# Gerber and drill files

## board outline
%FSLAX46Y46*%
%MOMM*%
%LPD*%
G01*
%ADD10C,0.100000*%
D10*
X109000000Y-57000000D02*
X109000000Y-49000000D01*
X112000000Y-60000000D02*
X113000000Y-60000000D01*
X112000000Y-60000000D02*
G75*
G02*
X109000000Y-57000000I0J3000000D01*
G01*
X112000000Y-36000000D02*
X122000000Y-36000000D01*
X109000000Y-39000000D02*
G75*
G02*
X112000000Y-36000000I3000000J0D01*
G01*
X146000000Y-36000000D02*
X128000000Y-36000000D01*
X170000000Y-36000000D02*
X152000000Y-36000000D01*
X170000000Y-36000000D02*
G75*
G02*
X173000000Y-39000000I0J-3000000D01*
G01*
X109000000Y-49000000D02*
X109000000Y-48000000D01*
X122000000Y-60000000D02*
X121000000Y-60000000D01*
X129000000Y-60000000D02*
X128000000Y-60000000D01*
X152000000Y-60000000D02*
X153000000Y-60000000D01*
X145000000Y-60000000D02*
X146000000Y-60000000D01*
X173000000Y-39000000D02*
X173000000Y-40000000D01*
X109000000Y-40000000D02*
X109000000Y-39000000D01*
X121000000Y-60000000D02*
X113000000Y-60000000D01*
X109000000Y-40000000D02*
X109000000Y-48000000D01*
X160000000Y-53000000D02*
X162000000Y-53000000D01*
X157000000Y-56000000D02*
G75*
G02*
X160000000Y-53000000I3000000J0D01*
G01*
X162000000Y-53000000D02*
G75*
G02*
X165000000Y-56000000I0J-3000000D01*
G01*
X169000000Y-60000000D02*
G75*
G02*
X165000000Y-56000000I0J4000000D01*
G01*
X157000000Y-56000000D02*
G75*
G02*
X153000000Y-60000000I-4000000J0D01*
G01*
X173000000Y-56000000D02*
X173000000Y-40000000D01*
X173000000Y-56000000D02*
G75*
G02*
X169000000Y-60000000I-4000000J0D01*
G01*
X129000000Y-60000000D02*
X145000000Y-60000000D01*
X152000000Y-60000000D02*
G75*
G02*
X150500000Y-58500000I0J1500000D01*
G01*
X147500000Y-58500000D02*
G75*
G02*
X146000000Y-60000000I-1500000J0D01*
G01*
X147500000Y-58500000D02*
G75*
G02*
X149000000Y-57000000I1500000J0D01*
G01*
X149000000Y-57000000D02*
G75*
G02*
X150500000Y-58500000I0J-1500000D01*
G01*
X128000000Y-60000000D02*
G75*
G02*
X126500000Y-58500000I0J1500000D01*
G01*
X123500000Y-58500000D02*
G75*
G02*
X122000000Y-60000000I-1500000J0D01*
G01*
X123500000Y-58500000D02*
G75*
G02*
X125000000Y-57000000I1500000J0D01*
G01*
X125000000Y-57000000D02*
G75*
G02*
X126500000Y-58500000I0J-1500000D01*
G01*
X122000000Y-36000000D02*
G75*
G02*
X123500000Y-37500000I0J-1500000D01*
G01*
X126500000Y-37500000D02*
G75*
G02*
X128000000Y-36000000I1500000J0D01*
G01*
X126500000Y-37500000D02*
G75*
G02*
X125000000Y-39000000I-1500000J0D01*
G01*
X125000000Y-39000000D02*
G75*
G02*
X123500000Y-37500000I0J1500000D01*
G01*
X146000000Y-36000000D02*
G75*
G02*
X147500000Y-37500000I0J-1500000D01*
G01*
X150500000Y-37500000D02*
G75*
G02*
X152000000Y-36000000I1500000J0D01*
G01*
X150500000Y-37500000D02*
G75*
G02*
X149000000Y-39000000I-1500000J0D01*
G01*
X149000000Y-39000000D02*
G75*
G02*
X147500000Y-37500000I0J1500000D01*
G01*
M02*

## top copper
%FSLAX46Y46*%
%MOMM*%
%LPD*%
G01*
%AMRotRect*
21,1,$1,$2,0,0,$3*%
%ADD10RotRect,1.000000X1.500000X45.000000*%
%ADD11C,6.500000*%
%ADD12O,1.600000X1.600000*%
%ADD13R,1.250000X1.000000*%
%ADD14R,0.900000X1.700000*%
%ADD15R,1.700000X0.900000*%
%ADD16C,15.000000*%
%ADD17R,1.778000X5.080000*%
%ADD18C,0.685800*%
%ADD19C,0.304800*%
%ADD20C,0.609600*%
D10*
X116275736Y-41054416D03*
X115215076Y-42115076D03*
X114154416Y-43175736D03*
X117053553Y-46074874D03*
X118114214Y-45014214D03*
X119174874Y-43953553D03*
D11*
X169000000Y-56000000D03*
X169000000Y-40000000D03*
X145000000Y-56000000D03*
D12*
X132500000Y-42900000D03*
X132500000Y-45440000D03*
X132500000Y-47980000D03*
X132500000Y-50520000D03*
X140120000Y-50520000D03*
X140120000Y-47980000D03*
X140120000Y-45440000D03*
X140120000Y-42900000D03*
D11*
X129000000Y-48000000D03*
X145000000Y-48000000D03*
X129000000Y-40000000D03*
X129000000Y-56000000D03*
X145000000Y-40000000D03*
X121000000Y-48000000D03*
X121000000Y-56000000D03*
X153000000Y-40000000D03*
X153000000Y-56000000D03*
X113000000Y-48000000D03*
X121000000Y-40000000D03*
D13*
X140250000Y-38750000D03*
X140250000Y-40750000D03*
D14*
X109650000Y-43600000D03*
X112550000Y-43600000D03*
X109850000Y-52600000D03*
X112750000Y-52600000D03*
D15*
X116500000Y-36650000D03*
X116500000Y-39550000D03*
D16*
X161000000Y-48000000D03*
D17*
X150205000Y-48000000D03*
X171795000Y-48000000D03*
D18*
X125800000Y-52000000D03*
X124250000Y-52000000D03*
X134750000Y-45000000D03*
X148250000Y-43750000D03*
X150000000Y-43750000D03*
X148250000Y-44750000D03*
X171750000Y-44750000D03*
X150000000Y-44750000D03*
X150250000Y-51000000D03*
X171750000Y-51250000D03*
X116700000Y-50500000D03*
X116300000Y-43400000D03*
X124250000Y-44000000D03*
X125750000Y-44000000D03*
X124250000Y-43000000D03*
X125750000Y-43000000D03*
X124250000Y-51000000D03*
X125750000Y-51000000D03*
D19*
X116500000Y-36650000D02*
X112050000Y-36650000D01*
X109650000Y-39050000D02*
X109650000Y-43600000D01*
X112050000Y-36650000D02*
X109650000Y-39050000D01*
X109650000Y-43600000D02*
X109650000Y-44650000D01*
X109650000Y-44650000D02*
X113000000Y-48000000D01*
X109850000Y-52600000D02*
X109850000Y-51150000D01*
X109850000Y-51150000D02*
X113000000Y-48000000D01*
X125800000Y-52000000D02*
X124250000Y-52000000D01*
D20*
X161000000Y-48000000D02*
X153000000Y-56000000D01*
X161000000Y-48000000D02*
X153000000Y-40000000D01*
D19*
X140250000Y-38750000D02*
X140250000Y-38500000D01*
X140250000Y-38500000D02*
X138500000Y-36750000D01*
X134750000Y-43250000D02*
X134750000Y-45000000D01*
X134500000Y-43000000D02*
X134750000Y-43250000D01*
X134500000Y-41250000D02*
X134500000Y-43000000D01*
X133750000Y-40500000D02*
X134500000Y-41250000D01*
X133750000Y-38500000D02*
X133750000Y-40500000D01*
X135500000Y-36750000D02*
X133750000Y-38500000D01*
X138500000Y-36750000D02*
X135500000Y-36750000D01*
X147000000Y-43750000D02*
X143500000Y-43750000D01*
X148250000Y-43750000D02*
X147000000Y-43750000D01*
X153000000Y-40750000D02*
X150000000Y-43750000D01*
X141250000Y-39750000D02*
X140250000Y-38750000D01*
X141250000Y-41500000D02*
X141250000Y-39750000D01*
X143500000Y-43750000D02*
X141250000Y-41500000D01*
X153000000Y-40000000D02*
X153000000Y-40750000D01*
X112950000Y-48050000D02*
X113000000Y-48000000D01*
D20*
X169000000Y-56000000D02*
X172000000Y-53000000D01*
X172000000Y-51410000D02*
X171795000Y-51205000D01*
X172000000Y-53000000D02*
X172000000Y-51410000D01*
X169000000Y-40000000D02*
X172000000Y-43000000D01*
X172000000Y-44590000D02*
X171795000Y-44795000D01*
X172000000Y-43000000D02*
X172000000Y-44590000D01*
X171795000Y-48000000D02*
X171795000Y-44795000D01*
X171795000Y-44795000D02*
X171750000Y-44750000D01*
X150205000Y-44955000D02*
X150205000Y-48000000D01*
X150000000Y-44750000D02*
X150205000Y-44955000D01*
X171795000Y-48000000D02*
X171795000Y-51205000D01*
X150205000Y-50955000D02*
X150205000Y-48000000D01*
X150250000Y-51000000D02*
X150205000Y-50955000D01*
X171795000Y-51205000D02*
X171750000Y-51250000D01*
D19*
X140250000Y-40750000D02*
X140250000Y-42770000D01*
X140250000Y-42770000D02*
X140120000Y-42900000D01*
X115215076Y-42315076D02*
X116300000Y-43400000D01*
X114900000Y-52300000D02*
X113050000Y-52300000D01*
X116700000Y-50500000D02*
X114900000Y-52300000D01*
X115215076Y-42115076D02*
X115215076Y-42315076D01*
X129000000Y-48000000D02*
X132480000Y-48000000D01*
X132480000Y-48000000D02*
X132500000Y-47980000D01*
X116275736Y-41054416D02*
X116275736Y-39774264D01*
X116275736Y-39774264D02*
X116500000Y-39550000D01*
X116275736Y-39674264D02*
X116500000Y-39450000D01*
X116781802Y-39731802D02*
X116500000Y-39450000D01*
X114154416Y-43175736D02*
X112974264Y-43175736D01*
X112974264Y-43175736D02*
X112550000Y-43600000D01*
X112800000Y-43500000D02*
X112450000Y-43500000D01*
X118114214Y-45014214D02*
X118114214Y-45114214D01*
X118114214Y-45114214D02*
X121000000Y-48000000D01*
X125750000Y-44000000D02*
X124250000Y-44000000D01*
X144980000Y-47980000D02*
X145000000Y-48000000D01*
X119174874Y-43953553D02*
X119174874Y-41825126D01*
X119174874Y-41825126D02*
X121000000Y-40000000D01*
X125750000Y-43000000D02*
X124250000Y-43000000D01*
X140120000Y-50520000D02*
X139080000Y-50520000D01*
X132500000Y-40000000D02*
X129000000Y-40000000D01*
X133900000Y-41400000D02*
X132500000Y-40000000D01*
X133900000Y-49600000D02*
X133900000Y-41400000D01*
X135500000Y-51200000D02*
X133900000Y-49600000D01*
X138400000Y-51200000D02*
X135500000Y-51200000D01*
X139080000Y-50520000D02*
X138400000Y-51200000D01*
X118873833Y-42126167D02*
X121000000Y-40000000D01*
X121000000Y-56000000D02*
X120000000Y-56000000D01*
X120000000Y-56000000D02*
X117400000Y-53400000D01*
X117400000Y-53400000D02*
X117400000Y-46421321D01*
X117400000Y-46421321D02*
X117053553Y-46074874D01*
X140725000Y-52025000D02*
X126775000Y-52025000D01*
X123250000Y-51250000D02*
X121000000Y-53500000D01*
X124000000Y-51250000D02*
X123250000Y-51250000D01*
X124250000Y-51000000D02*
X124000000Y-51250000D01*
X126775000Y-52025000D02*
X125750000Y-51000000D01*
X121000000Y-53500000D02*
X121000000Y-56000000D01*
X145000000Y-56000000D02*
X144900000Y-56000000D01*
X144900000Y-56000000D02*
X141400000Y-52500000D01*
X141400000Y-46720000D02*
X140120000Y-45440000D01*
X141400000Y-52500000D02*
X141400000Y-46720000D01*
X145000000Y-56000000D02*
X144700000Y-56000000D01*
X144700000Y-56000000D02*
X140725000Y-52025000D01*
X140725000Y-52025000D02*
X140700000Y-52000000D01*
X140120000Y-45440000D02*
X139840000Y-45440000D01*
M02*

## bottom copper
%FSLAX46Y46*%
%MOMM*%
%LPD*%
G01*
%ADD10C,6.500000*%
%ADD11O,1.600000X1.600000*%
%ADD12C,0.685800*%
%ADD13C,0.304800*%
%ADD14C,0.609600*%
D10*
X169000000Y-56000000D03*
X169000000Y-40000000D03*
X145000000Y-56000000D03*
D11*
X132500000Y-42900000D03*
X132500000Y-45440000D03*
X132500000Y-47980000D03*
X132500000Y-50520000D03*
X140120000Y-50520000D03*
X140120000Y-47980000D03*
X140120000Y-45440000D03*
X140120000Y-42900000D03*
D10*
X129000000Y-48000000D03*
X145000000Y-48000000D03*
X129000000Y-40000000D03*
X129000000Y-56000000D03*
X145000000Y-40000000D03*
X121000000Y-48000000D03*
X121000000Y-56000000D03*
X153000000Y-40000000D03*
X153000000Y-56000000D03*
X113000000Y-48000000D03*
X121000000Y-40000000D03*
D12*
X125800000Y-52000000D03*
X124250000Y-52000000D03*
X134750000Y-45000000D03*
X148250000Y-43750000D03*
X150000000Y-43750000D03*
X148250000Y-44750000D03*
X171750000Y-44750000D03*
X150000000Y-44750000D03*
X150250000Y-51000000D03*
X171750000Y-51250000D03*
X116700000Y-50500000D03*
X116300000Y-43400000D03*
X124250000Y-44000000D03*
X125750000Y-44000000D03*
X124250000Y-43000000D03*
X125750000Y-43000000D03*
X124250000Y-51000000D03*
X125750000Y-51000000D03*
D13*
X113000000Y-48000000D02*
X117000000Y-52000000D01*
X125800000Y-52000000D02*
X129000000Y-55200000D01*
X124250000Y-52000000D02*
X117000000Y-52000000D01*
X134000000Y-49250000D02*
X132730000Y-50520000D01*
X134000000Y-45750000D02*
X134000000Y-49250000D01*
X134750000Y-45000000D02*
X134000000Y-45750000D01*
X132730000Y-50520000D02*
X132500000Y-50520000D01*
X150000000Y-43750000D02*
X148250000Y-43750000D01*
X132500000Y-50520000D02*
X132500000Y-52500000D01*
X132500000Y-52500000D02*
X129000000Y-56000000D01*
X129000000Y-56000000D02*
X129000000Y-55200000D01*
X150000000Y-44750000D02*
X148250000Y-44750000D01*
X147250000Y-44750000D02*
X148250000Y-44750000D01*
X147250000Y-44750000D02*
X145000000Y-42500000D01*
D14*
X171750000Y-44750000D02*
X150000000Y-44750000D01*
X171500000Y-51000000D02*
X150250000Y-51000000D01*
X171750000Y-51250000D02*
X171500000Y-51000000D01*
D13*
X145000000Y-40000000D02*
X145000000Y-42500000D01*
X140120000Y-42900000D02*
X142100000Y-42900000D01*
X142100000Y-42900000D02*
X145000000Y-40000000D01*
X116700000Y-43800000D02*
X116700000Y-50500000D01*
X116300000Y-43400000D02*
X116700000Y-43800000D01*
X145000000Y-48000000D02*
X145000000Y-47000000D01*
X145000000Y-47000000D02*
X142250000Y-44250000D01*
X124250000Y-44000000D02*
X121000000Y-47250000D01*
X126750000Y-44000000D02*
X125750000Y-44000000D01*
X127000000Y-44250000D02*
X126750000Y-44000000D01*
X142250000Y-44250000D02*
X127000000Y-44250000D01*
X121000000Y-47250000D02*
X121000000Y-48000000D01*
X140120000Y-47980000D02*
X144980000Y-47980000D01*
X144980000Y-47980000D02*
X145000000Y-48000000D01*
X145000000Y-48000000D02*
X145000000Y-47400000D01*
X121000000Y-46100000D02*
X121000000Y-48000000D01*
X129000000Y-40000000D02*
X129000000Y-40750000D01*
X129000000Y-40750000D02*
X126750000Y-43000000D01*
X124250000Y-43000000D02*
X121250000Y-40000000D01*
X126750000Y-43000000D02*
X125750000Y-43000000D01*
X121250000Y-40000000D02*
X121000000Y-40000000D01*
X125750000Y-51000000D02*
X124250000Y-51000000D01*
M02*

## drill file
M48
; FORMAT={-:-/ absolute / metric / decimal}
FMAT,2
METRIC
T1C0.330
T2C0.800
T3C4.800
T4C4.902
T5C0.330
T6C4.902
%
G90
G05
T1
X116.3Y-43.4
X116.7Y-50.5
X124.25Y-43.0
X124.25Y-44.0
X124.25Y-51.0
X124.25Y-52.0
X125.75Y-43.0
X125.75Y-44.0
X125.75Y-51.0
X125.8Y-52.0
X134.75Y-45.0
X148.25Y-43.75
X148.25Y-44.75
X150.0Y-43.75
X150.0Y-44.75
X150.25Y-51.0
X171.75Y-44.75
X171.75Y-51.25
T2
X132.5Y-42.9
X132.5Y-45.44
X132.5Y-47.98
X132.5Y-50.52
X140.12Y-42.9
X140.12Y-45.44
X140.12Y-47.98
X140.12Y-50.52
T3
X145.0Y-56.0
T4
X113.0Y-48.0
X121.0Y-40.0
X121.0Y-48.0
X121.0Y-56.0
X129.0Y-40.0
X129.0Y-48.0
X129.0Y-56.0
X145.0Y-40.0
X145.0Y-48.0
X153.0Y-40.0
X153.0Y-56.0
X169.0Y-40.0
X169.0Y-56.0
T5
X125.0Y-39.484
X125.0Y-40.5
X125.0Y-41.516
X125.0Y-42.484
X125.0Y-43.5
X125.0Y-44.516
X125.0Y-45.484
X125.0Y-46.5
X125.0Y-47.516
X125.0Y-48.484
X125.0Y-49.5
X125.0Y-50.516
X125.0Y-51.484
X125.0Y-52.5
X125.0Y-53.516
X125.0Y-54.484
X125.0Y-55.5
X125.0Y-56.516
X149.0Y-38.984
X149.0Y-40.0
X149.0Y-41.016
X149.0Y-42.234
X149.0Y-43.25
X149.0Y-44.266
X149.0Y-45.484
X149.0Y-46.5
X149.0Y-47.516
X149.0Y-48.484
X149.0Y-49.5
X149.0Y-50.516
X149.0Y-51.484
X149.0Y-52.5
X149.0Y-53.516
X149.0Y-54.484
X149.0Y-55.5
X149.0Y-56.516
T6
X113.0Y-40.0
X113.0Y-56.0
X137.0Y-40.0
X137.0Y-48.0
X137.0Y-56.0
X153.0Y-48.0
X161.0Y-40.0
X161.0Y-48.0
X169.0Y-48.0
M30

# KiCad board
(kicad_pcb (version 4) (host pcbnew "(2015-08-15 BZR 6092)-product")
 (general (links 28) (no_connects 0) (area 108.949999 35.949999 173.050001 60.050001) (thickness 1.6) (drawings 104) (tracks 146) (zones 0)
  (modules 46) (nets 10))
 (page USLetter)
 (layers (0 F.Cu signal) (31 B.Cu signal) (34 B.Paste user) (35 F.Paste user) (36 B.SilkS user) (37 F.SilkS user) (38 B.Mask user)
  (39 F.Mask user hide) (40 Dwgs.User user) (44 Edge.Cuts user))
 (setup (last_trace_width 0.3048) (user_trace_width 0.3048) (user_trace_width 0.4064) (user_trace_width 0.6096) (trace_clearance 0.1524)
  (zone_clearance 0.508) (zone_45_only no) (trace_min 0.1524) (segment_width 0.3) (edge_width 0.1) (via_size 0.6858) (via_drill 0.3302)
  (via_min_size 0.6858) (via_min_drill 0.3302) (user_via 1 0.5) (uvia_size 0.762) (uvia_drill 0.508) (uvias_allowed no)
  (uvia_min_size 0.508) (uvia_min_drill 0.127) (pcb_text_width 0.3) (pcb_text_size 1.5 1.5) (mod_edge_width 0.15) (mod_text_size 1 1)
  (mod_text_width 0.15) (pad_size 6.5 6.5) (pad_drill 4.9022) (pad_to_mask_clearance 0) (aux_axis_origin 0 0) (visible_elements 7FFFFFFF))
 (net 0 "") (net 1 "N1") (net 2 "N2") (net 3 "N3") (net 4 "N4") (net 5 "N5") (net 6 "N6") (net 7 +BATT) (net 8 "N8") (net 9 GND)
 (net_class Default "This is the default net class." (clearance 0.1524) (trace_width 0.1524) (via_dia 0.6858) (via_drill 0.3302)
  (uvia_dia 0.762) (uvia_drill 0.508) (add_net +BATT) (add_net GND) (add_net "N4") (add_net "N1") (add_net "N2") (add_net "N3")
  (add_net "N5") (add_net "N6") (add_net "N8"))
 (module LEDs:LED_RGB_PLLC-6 (layer F.Cu) (at 116.7 43.6 315)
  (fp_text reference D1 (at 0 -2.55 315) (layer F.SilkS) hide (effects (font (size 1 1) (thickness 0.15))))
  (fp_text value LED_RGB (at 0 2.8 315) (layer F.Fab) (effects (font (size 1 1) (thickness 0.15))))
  (pad 1 smd rect (at -2.1 -1.5 45) (size 1 1.5) (layers F.Cu F.Paste F.Mask) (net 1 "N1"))
  (pad 2 smd rect (at -2.1 0 45) (size 1 1.5) (layers F.Cu F.Paste F.Mask) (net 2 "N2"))
  (pad 3 smd rect (at -2.1 1.5 45) (size 1 1.5) (layers F.Cu F.Paste F.Mask) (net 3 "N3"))
  (pad 4 smd rect (at 2 1.5 45) (size 1 1.5) (layers F.Cu F.Paste F.Mask) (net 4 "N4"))
  (pad 5 smd rect (at 2 0 45) (size 1 1.5) (layers F.Cu F.Paste F.Mask) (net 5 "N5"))
  (pad 6 smd rect (at 2 -1.5 45) (size 1 1.5) (layers F.Cu F.Paste F.Mask) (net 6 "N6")))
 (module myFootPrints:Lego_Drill (layer F.Cu) (at 113 40)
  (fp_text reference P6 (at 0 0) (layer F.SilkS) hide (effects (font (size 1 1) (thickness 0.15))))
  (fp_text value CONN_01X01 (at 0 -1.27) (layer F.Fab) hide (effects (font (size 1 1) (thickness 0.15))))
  (pad "" np_thru_hole circle (at 0 0) (size 4.9022 4.9022) (drill 4.9022) (layers *.Cu *.Mask F.SilkS)))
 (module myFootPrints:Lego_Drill (layer F.Cu) (at 113 56)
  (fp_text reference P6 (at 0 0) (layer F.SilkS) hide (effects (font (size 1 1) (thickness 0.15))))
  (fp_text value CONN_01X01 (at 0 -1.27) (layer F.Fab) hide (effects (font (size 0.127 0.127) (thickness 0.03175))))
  (pad "" np_thru_hole circle (at 0 0) (size 4.9022 4.9022) (drill 4.9022) (layers *.Cu *.Mask F.SilkS)))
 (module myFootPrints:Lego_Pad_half (layer F.Cu) (at 169 56 180)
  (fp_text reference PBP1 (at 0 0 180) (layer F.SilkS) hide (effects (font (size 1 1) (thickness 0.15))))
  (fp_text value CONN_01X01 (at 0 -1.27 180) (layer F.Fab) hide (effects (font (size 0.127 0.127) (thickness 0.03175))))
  (pad 1 thru_hole circle (at 0 0 180) (size 6.5 6.5) (drill 4.9022) (layers *.Cu B.Mask) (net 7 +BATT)))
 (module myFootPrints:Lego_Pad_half (layer F.Cu) (at 169 40 270)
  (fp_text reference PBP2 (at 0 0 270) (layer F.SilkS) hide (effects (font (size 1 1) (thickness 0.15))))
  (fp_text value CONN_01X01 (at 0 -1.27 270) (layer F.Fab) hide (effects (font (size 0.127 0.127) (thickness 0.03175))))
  (pad 1 thru_hole circle (at 0 0 270) (size 6.5 6.5) (drill 4.9022) (layers *.Cu B.Mask) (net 7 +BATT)))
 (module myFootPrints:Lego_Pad (layer F.Cu) (at 145 56)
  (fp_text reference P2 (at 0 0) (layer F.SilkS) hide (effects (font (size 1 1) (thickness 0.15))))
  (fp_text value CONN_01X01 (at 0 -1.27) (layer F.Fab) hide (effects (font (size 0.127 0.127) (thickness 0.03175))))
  (pad 1 thru_hole circle (at 0 0) (size 6.5 6.5) (drill 4.8) (layers *.Cu *.Mask F.SilkS) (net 4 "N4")))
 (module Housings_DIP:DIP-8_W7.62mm (layer F.Cu) (at 132.5 42.9)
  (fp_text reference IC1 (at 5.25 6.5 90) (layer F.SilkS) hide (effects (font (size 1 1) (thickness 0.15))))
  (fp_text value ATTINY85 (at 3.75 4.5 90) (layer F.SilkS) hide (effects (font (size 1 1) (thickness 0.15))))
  (pad 1 thru_hole oval (at 0 0) (size 1.6 1.6) (drill 0.8) (layers *.Cu *.Mask F.SilkS))
  (pad 2 thru_hole oval (at 0 2.54) (size 1.6 1.6) (drill 0.8) (layers *.Cu *.Mask F.SilkS))
  (pad 3 thru_hole oval (at 0 5.08) (size 1.6 1.6) (drill 0.8) (layers *.Cu *.Mask F.SilkS) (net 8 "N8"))
  (pad 4 thru_hole oval (at 0 7.62) (size 1.6 1.6) (drill 0.8) (layers *.Cu *.Mask F.SilkS) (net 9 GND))
  (pad 5 thru_hole oval (at 7.62 7.62) (size 1.6 1.6) (drill 0.8) (layers *.Cu *.Mask F.SilkS) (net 6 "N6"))
  (pad 6 thru_hole oval (at 7.62 5.08) (size 1.6 1.6) (drill 0.8) (layers *.Cu *.Mask F.SilkS) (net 5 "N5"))
  (pad 7 thru_hole oval (at 7.62 2.54) (size 1.6 1.6) (drill 0.8) (layers *.Cu *.Mask F.SilkS) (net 4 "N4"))
  (pad 8 thru_hole oval (at 7.62 0) (size 1.6 1.6) (drill 0.8) (layers *.Cu *.Mask F.SilkS) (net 7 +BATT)))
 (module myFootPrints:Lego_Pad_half (layer F.Cu) (at 129 48 45)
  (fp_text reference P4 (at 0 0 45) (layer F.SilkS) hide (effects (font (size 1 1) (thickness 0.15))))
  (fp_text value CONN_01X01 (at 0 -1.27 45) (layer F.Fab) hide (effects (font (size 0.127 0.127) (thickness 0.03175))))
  (pad 1 thru_hole circle (at 0 0 45) (size 6.5 6.5) (drill 4.9022) (layers *.Cu *.Mask F.SilkS) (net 8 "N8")))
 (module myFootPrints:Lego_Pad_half (layer F.Cu) (at 145 48 225)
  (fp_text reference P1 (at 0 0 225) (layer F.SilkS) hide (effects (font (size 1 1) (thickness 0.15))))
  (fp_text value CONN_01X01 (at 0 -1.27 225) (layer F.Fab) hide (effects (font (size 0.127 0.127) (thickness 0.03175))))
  (pad 1 thru_hole circle (at 0 0 225) (size 6.5 6.5) (drill 4.9022) (layers *.Cu *.Mask F.SilkS) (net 5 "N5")))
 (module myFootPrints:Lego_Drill (layer F.Cu) (at 137 40)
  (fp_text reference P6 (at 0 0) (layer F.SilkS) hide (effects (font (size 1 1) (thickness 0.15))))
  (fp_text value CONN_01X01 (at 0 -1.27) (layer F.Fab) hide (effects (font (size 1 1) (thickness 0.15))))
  (pad "" np_thru_hole circle (at 0 0) (size 4.9022 4.9022) (drill 4.9022) (layers *.Cu *.Mask F.SilkS)))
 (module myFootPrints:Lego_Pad (layer F.Cu) (at 129 40)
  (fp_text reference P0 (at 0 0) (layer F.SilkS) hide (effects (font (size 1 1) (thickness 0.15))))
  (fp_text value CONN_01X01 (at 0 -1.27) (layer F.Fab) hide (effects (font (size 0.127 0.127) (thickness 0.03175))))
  (pad 1 thru_hole circle (at 0 0) (size 6.5 6.5) (drill 4.9022) (layers *.Cu *.Mask F.SilkS) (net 6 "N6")))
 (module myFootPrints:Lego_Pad (layer F.Cu) (at 129 56)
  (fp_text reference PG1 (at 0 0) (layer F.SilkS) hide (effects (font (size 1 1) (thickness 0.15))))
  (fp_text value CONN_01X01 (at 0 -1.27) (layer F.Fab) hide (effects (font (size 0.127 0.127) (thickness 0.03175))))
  (pad 1 thru_hole circle (at 0 0) (size 6.5 6.5) (drill 4.9022) (layers *.Cu *.Mask F.SilkS) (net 9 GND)))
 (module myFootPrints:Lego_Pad (layer F.Cu) (at 145 40)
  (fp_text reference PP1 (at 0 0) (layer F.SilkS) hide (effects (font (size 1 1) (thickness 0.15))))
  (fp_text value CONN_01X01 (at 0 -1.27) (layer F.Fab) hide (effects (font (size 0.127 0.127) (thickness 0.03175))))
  (pad 1 thru_hole circle (at 0 0) (size 6.5 6.5) (drill 4.9022) (layers *.Cu *.Mask F.SilkS) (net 7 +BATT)))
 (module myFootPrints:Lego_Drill (layer F.Cu) (at 137 48)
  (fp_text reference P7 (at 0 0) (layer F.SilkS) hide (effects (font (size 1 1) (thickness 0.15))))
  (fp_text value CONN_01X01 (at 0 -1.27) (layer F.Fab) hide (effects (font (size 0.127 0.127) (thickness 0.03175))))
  (pad "" np_thru_hole circle (at 0 0) (size 4.9022 4.9022) (drill 4.9022) (layers *.Cu *.Mask F.SilkS)))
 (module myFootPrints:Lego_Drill (layer F.Cu) (at 137 56)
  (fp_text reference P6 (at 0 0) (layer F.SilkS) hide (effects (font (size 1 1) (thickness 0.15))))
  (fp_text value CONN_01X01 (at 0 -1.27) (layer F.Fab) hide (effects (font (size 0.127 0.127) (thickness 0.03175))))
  (pad "" np_thru_hole circle (at 0 0) (size 4.9022 4.9022) (drill 4.9022) (layers *.Cu *.Mask F.SilkS)))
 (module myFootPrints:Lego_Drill (layer F.Cu) (at 161 48)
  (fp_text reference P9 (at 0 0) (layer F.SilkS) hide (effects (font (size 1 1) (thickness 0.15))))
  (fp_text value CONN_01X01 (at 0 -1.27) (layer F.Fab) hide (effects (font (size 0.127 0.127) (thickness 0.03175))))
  (pad "" np_thru_hole circle (at 0 0) (size 4.9022 4.9022) (drill 4.9022) (layers *.Cu *.Mask F.SilkS)))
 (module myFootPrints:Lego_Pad (layer F.Cu) (at 121 48)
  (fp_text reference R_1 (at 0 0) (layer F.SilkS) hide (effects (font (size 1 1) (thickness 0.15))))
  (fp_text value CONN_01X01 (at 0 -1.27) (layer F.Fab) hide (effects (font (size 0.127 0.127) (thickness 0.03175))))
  (pad 1 thru_hole circle (at 0 0) (size 6.5 6.5) (drill 4.9022) (layers *.Cu *.Mask F.SilkS) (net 5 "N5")))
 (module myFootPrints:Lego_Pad (layer F.Cu) (at 121 56)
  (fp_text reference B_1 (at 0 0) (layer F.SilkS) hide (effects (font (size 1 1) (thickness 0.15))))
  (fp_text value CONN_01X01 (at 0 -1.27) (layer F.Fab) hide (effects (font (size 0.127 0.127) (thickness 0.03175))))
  (pad 1 thru_hole circle (at 0 0) (size 6.5 6.5) (drill 4.9022) (layers *.Cu *.Mask F.SilkS) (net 4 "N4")))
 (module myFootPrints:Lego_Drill (layer F.Cu) (at 169 48)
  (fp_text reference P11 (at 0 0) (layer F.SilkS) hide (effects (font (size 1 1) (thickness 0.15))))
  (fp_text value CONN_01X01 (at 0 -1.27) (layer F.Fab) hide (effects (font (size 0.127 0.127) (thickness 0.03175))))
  (pad "" np_thru_hole circle (at 0 0) (size 4.9022 4.9022) (drill 4.9022) (layers *.Cu *.Mask F.SilkS)))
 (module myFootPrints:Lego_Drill (layer F.Cu) (at 153 48)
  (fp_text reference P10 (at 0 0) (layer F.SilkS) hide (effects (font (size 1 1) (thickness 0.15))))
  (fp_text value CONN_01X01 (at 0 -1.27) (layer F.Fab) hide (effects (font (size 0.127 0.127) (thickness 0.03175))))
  (pad "" np_thru_hole circle (at 0 0) (size 4.9022 4.9022) (drill 4.9022) (layers *.Cu *.Mask F.SilkS)))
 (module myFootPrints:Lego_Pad (layer F.Cu) (at 153 40)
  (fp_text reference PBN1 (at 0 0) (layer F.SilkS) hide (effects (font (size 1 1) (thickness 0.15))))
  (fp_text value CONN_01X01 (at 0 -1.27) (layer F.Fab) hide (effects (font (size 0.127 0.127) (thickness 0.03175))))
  (pad 1 thru_hole circle (at 0 0) (size 6.5 6.5) (drill 4.9022) (layers *.Cu *.Mask F.SilkS) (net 9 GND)))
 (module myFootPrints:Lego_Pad (layer F.Cu) (at 153 56)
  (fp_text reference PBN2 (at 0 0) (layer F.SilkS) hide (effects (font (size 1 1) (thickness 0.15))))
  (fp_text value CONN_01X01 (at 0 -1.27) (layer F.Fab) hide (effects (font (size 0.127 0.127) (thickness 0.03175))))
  (pad 1 thru_hole circle (at 0 0) (size 6.5 6.5) (drill 4.9022) (layers *.Cu *.Mask F.SilkS) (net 9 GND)))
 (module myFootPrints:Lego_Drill (layer F.Cu) (at 161 40)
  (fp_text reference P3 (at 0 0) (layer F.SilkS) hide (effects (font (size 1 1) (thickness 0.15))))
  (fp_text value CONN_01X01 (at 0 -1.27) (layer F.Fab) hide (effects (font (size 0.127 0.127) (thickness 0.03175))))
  (pad "" np_thru_hole circle (at 0 0) (size 4.9022 4.9022) (drill 4.9022) (layers *.Cu *.Mask F.SilkS)))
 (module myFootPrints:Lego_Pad (layer F.Cu) (at 113 48)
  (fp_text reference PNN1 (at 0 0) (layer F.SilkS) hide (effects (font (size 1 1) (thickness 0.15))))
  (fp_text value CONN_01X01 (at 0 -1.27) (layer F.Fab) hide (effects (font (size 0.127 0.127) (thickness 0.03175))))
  (pad 1 thru_hole circle (at 0 0) (size 6.5 6.5) (drill 4.9022) (layers *.Cu *.Mask F.SilkS) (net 9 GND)))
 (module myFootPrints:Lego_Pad (layer F.Cu) (at 121 40)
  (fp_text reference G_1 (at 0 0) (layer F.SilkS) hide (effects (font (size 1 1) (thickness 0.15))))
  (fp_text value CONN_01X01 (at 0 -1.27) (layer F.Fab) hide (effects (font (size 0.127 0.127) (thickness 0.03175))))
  (pad 1 thru_hole circle (at 0 0) (size 6.5 6.5) (drill 4.9022) (layers *.Cu *.Mask F.SilkS) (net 6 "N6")))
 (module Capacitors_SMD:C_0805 (layer F.Cu) (at 140.25 39.75 270)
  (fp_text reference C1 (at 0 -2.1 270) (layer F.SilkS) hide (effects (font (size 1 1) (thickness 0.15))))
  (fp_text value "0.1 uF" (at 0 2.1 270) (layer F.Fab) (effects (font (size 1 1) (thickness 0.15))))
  (pad 1 smd rect (at -1 0 270) (size 1 1.25) (layers F.Cu F.Paste F.Mask) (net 9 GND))
  (pad 2 smd rect (at 1 0 270) (size 1 1.25) (layers F.Cu F.Paste F.Mask) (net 7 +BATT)))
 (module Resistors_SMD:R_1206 (layer F.Cu) (at 111.1 43.6)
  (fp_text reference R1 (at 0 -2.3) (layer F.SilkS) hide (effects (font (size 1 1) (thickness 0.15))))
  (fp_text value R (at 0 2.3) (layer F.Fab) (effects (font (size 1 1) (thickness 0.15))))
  (pad 1 smd rect (at -1.45 0) (size 0.9 1.7) (layers F.Cu F.Paste F.Mask) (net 9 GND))
  (pad 2 smd rect (at 1.45 0) (size 0.9 1.7) (layers F.Cu F.Paste F.Mask) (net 3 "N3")))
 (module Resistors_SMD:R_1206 (layer F.Cu) (at 111.3 52.6)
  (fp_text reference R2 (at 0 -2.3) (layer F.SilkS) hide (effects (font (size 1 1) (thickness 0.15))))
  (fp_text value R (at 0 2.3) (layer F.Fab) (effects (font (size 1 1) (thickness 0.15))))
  (pad 1 smd rect (at -1.45 0) (size 0.9 1.7) (layers F.Cu F.Paste F.Mask) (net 9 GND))
  (pad 2 smd rect (at 1.45 0) (size 0.9 1.7) (layers F.Cu F.Paste F.Mask) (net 2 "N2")))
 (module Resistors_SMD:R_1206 (layer F.Cu) (at 116.5 38.1 270)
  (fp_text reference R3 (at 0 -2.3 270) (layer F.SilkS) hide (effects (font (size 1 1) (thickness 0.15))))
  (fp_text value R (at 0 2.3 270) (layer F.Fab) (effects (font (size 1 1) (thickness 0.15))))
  (pad 1 smd rect (at -1.45 0 270) (size 0.9 1.7) (layers F.Cu F.Paste F.Mask) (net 9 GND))
  (pad 2 smd rect (at 1.45 0 270) (size 0.9 1.7) (layers F.Cu F.Paste F.Mask) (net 1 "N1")))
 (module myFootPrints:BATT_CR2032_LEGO (layer F.Cu) (at 161 48)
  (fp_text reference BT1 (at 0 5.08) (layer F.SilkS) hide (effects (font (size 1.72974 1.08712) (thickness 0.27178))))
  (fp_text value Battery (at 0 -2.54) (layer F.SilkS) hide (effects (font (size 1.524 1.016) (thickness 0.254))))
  (pad 2 smd circle (at 0 0) (size 15 15) (layers F.Cu F.Paste F.Mask) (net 9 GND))
  (pad 1 smd rect (at -10.795 0) (size 1.778 5.08) (layers F.Cu F.Paste F.Mask) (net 7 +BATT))
  (pad 1 smd rect (at 10.795 0) (size 1.778 5.08) (layers F.Cu F.Paste F.Mask) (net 7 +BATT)))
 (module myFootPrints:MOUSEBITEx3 (layer F.Cu) (at 149 40 90)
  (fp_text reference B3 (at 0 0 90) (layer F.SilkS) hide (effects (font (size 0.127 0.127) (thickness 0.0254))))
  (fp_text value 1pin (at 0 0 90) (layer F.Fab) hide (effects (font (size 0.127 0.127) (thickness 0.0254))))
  (pad "" np_thru_hole circle (at -1.016 0 90) (size 0.3302 0.3302) (drill 0.3302) (layers *.Cu *.Mask F.SilkS))
  (pad "" np_thru_hole circle (at 1.016 0 90) (size 0.3302 0.3302) (drill 0.3302) (layers *.Cu *.Mask F.SilkS))
  (pad "" np_thru_hole circle (at 0 0 90) (size 0.3302 0.3302) (drill 0.3302) (layers *.Cu *.Mask F.SilkS)))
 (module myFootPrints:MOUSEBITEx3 (layer F.Cu) (at 149 49.5 90)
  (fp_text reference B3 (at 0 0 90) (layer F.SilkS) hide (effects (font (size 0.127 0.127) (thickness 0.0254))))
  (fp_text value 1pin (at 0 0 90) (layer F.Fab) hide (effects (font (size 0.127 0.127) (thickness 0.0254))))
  (pad "" np_thru_hole circle (at -1.016 0 90) (size 0.3302 0.3302) (drill 0.3302) (layers *.Cu *.Mask F.SilkS))
  (pad "" np_thru_hole circle (at 1.016 0 90) (size 0.3302 0.3302) (drill 0.3302) (layers *.Cu *.Mask F.SilkS))
  (pad "" np_thru_hole circle (at 0 0 90) (size 0.3302 0.3302) (drill 0.3302) (layers *.Cu *.Mask F.SilkS)))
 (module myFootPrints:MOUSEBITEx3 (layer F.Cu) (at 149 52.5 90)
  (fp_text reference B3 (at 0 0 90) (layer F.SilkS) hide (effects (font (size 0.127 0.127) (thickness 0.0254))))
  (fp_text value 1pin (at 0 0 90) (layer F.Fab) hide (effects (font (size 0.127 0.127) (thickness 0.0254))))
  (pad "" np_thru_hole circle (at -1.016 0 90) (size 0.3302 0.3302) (drill 0.3302) (layers *.Cu *.Mask F.SilkS))
  (pad "" np_thru_hole circle (at 1.016 0 90) (size 0.3302 0.3302) (drill 0.3302) (layers *.Cu *.Mask F.SilkS))
  (pad "" np_thru_hole circle (at 0 0 90) (size 0.3302 0.3302) (drill 0.3302) (layers *.Cu *.Mask F.SilkS)))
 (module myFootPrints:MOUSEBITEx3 (layer F.Cu) (at 149 55.5 90)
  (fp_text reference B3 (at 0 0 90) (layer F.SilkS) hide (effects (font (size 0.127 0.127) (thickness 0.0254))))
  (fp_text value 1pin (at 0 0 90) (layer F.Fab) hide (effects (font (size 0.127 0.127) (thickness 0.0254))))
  (pad "" np_thru_hole circle (at -1.016 0 90) (size 0.3302 0.3302) (drill 0.3302) (layers *.Cu *.Mask F.SilkS))
  (pad "" np_thru_hole circle (at 1.016 0 90) (size 0.3302 0.3302) (drill 0.3302) (layers *.Cu *.Mask F.SilkS))
  (pad "" np_thru_hole circle (at 0 0 90) (size 0.3302 0.3302) (drill 0.3302) (layers *.Cu *.Mask F.SilkS)))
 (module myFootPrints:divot (layer F.Cu) (at 149 60 180)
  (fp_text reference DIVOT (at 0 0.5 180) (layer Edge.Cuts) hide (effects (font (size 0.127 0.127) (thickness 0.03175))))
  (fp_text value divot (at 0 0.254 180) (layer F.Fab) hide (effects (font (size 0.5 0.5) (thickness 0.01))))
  (fp_arc (start -3 1.5) (end -3 0) (angle 90) (layer Edge.Cuts) (width 0.1))
  (fp_arc (start 3 1.5) (end 1.5 1.5) (angle 90) (layer Edge.Cuts) (width 0.1))
  (fp_arc (start 0 1.5) (end 1.5 1.5) (angle 90) (layer Edge.Cuts) (width 0.1))
  (fp_arc (start 0 1.5) (end 0 3) (angle 90) (layer Edge.Cuts) (width 0.1)))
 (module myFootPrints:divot (layer F.Cu) (at 125 60 180)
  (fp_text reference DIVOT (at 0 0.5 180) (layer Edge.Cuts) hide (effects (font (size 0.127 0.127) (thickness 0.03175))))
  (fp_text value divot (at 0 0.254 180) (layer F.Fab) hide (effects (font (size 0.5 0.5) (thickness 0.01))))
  (fp_arc (start -3 1.5) (end -3 0) (angle 90) (layer Edge.Cuts) (width 0.1))
  (fp_arc (start 3 1.5) (end 1.5 1.5) (angle 90) (layer Edge.Cuts) (width 0.1))
  (fp_arc (start 0 1.5) (end 1.5 1.5) (angle 90) (layer Edge.Cuts) (width 0.1))
  (fp_arc (start 0 1.5) (end 0 3) (angle 90) (layer Edge.Cuts) (width 0.1)))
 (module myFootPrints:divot (layer F.Cu) (at 125 36)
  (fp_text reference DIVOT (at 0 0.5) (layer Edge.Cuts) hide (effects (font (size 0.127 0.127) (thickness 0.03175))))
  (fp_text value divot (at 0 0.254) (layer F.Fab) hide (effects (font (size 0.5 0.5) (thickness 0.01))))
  (fp_arc (start -3 1.5) (end -3 0) (angle 90) (layer Edge.Cuts) (width 0.1))
  (fp_arc (start 3 1.5) (end 1.5 1.5) (angle 90) (layer Edge.Cuts) (width 0.1))
  (fp_arc (start 0 1.5) (end 1.5 1.5) (angle 90) (layer Edge.Cuts) (width 0.1))
  (fp_arc (start 0 1.5) (end 0 3) (angle 90) (layer Edge.Cuts) (width 0.1)))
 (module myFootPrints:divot (layer F.Cu) (at 149 36)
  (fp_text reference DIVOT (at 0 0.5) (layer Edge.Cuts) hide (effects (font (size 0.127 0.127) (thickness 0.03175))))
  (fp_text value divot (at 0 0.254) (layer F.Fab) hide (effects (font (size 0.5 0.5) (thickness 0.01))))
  (fp_arc (start -3 1.5) (end -3 0) (angle 90) (layer Edge.Cuts) (width 0.1))
  (fp_arc (start 3 1.5) (end 1.5 1.5) (angle 90) (layer Edge.Cuts) (width 0.1))
  (fp_arc (start 0 1.5) (end 1.5 1.5) (angle 90) (layer Edge.Cuts) (width 0.1))
  (fp_arc (start 0 1.5) (end 0 3) (angle 90) (layer Edge.Cuts) (width 0.1)))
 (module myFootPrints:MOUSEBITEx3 (layer F.Cu) (at 149 46.5 90)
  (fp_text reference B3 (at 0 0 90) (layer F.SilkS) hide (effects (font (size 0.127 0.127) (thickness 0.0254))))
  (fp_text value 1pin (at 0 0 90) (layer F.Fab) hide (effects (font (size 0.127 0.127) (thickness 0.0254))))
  (pad "" np_thru_hole circle (at -1.016 0 90) (size 0.3302 0.3302) (drill 0.3302) (layers *.Cu *.Mask F.SilkS))
  (pad "" np_thru_hole circle (at 1.016 0 90) (size 0.3302 0.3302) (drill 0.3302) (layers *.Cu *.Mask F.SilkS))
  (pad "" np_thru_hole circle (at 0 0 90) (size 0.3302 0.3302) (drill 0.3302) (layers *.Cu *.Mask F.SilkS)))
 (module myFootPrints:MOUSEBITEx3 (layer F.Cu) (at 149 43.25 90)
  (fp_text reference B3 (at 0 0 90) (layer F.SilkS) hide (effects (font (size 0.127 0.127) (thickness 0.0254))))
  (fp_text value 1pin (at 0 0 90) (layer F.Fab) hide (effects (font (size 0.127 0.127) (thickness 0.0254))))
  (pad "" np_thru_hole circle (at -1.016 0 90) (size 0.3302 0.3302) (drill 0.3302) (layers *.Cu *.Mask F.SilkS))
  (pad "" np_thru_hole circle (at 1.016 0 90) (size 0.3302 0.3302) (drill 0.3302) (layers *.Cu *.Mask F.SilkS))
  (pad "" np_thru_hole circle (at 0 0 90) (size 0.3302 0.3302) (drill 0.3302) (layers *.Cu *.Mask F.SilkS)))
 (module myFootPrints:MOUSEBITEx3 (layer F.Cu) (at 125 55.5 90)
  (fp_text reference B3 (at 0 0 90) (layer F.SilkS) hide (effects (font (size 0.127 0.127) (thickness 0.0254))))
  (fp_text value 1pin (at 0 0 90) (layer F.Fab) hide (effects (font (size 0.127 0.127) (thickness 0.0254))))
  (pad "" np_thru_hole circle (at -1.016 0 90) (size 0.3302 0.3302) (drill 0.3302) (layers *.Cu *.Mask F.SilkS))
  (pad "" np_thru_hole circle (at 1.016 0 90) (size 0.3302 0.3302) (drill 0.3302) (layers *.Cu *.Mask F.SilkS))
  (pad "" np_thru_hole circle (at 0 0 90) (size 0.3302 0.3302) (drill 0.3302) (layers *.Cu *.Mask F.SilkS)))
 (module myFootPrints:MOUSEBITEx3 (layer F.Cu) (at 125 52.5 90)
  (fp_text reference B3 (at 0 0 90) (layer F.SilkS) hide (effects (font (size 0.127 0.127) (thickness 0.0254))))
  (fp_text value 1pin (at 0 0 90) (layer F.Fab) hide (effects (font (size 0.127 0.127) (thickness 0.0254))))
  (pad "" np_thru_hole circle (at -1.016 0 90) (size 0.3302 0.3302) (drill 0.3302) (layers *.Cu *.Mask F.SilkS))
  (pad "" np_thru_hole circle (at 1.016 0 90) (size 0.3302 0.3302) (drill 0.3302) (layers *.Cu *.Mask F.SilkS))
  (pad "" np_thru_hole circle (at 0 0 90) (size 0.3302 0.3302) (drill 0.3302) (layers *.Cu *.Mask F.SilkS)))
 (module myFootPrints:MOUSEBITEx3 (layer F.Cu) (at 125 49.5 90)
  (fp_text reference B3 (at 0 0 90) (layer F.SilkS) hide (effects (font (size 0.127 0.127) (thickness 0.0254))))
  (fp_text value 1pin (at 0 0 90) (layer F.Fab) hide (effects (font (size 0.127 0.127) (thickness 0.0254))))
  (pad "" np_thru_hole circle (at -1.016 0 90) (size 0.3302 0.3302) (drill 0.3302) (layers *.Cu *.Mask F.SilkS))
  (pad "" np_thru_hole circle (at 1.016 0 90) (size 0.3302 0.3302) (drill 0.3302) (layers *.Cu *.Mask F.SilkS))
  (pad "" np_thru_hole circle (at 0 0 90) (size 0.3302 0.3302) (drill 0.3302) (layers *.Cu *.Mask F.SilkS)))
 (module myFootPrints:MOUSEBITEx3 (layer F.Cu) (at 125 46.5 90)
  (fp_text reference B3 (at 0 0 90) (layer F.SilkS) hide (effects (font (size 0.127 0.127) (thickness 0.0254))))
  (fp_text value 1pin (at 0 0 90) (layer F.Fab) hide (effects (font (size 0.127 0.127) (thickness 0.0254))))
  (pad "" np_thru_hole circle (at -1.016 0 90) (size 0.3302 0.3302) (drill 0.3302) (layers *.Cu *.Mask F.SilkS))
  (pad "" np_thru_hole circle (at 1.016 0 90) (size 0.3302 0.3302) (drill 0.3302) (layers *.Cu *.Mask F.SilkS))
  (pad "" np_thru_hole circle (at 0 0 90) (size 0.3302 0.3302) (drill 0.3302) (layers *.Cu *.Mask F.SilkS)))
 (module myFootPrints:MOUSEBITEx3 (layer F.Cu) (at 125 43.5 90)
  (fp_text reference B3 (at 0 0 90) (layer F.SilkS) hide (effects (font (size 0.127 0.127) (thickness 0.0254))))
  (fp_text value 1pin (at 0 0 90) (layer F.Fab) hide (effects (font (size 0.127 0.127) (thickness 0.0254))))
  (pad "" np_thru_hole circle (at -1.016 0 90) (size 0.3302 0.3302) (drill 0.3302) (layers *.Cu *.Mask F.SilkS))
  (pad "" np_thru_hole circle (at 1.016 0 90) (size 0.3302 0.3302) (drill 0.3302) (layers *.Cu *.Mask F.SilkS))
  (pad "" np_thru_hole circle (at 0 0 90) (size 0.3302 0.3302) (drill 0.3302) (layers *.Cu *.Mask F.SilkS)))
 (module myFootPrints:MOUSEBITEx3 (layer F.Cu) (at 125 40.5 90)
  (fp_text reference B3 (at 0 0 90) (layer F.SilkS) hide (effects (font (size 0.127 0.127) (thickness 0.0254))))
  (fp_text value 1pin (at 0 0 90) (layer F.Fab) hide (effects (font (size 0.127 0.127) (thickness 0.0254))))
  (pad "" np_thru_hole circle (at -1.016 0 90) (size 0.3302 0.3302) (drill 0.3302) (layers *.Cu *.Mask F.SilkS))
  (pad "" np_thru_hole circle (at 1.016 0 90) (size 0.3302 0.3302) (drill 0.3302) (layers *.Cu *.Mask F.SilkS))
  (pad "" np_thru_hole circle (at 0 0 90) (size 0.3302 0.3302) (drill 0.3302) (layers *.Cu *.Mask F.SilkS)))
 (gr_line (start 109 57) (end 109 49) (angle 90) (layer Edge.Cuts) (width 0.1))
 (gr_line (start 112 60) (end 113 60) (angle 90) (layer Edge.Cuts) (width 0.1))
 (gr_arc (start 112 57) (end 112 60) (angle 90) (layer Edge.Cuts) (width 0.1))
 (gr_line (start 112 36) (end 122 36) (angle 90) (layer Edge.Cuts) (width 0.1))
 (gr_arc (start 112 39) (end 109 39) (angle 90) (layer Edge.Cuts) (width 0.1))
 (gr_line (start 146 36) (end 128 36) (angle 90) (layer Edge.Cuts) (width 0.1))
 (gr_line (start 170 36) (end 152 36) (angle 90) (layer Edge.Cuts) (width 0.1))
 (gr_arc (start 170 39) (end 170 36) (angle 90) (layer Edge.Cuts) (width 0.1))
 (gr_line (start 109 49) (end 109 48) (angle 90) (layer Edge.Cuts) (width 0.1))
 (gr_line (start 122 60) (end 121 60) (angle 90) (layer Edge.Cuts) (width 0.1))
 (gr_line (start 129 60) (end 128 60) (angle 90) (layer Edge.Cuts) (width 0.1))
 (gr_line (start 152 60) (end 153 60) (angle 90) (layer Edge.Cuts) (width 0.1))
 (gr_line (start 145 60) (end 146 60) (angle 90) (layer Edge.Cuts) (width 0.1))
 (gr_line (start 173 39) (end 173 40) (angle 90) (layer Edge.Cuts) (width 0.1))
 (gr_line (start 109 40) (end 109 39) (angle 90) (layer Edge.Cuts) (width 0.1))
 (gr_line (start 121 60) (end 113 60) (angle 90) (layer Edge.Cuts) (width 0.1))
 (gr_line (start 109 40) (end 109 48) (angle 90) (layer Edge.Cuts) (width 0.1))
 (gr_line (start 160 53) (end 162 53) (angle 90) (layer Edge.Cuts) (width 0.1))
 (gr_arc (start 160 56) (end 157 56) (angle 90) (layer Edge.Cuts) (width 0.1))
 (gr_arc (start 162 56) (end 162 53) (angle 90) (layer Edge.Cuts) (width 0.1))
 (gr_arc (start 169 56) (end 169 60) (angle 90) (layer Edge.Cuts) (width 0.1))
 (gr_arc (start 153 56) (end 157 56) (angle 90) (layer Edge.Cuts) (width 0.1))
 (gr_line (start 173 56) (end 173 40) (angle 90) (layer Edge.Cuts) (width 0.1))
 (gr_arc (start 169 56) (end 173 56) (angle 90) (layer Edge.Cuts) (width 0.1))
 (gr_line (start 129 60) (end 145 60) (angle 90) (layer Edge.Cuts) (width 0.1))
 (segment (start 116.5 36.65) (end 112.05 36.65) (width 0.3048) (layer F.Cu) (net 9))
 (segment (start 109.65 39.05) (end 109.65 43.6) (width 0.3048) (layer F.Cu) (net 9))
 (segment (start 112.05 36.65) (end 109.65 39.05) (width 0.3048) (layer F.Cu) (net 9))
 (segment (start 109.65 43.6) (end 109.65 44.65) (width 0.3048) (layer F.Cu) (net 9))
 (segment (start 109.65 44.65) (end 113 48) (width 0.3048) (layer F.Cu) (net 9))
 (segment (start 109.85 52.6) (end 109.85 51.15) (width 0.3048) (layer F.Cu) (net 9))
 (segment (start 109.85 51.15) (end 113 48) (width 0.3048) (layer F.Cu) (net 9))
 (via (at 125.8 52) (size 0.6858) (drill 0.3302) (layers F.Cu B.Cu) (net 9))
 (segment (start 113 48) (end 117 52) (width 0.3048) (layer B.Cu) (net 9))
 (segment (start 125.8 52) (end 129 55.2) (width 0.3048) (layer B.Cu) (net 9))
 (segment (start 124.25 52) (end 117 52) (width 0.3048) (layer B.Cu) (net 9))
 (via (at 124.25 52) (size 0.6858) (drill 0.3302) (layers F.Cu B.Cu) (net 9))
 (segment (start 125.8 52) (end 124.25 52) (width 0.3048) (layer F.Cu) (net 9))
 (segment (start 161 48) (end 153 56) (width 0.6096) (layer F.Cu) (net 9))
 (segment (start 161 48) (end 153 40) (width 0.6096) (layer F.Cu) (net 9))
 (segment (start 140.25 38.75) (end 140.25 38.5) (width 0.3048) (layer F.Cu) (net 9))
 (segment (start 140.25 38.5) (end 138.5 36.75) (width 0.3048) (layer F.Cu) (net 9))
 (segment (start 134 49.25) (end 132.73 50.52) (width 0.3048) (layer B.Cu) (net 9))
 (segment (start 134 45.75) (end 134 49.25) (width 0.3048) (layer B.Cu) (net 9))
 (segment (start 134.75 45) (end 134 45.75) (width 0.3048) (layer B.Cu) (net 9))
 (via (at 134.75 45) (size 0.6858) (drill 0.3302) (layers F.Cu B.Cu) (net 9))
 (segment (start 134.75 43.25) (end 134.75 45) (width 0.3048) (layer F.Cu) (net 9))
 (segment (start 134.5 43) (end 134.75 43.25) (width 0.3048) (layer F.Cu) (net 9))
 (segment (start 134.5 41.25) (end 134.5 43) (width 0.3048) (layer F.Cu) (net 9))
 (segment (start 133.75 40.5) (end 134.5 41.25) (width 0.3048) (layer F.Cu) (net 9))
 (segment (start 133.75 38.5) (end 133.75 40.5) (width 0.3048) (layer F.Cu) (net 9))
 (segment (start 135.5 36.75) (end 133.75 38.5) (width 0.3048) (layer F.Cu) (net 9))
 (segment (start 138.5 36.75) (end 135.5 36.75) (width 0.3048) (layer F.Cu) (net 9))
 (segment (start 132.73 50.52) (end 132.5 50.52) (width 0.3048) (layer B.Cu) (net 9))
 (segment (start 147 43.75) (end 143.5 43.75) (width 0.3048) (layer F.Cu) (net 9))
 (segment (start 148.25 43.75) (end 147 43.75) (width 0.3048) (layer F.Cu) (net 9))
 (via (at 148.25 43.75) (size 0.6858) (drill 0.3302) (layers F.Cu B.Cu) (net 9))
 (segment (start 150 43.75) (end 148.25 43.75) (width 0.3048) (layer B.Cu) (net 9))
 (via (at 150 43.75) (size 0.6858) (drill 0.3302) (layers F.Cu B.Cu) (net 9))
 (segment (start 153 40.75) (end 150 43.75) (width 0.3048) (layer F.Cu) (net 9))
 (segment (start 141.25 39.75) (end 140.25 38.75) (width 0.3048) (layer F.Cu) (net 9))
 (segment (start 141.25 41.5) (end 141.25 39.75) (width 0.3048) (layer F.Cu) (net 9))
 (segment (start 143.5 43.75) (end 141.25 41.5) (width 0.3048) (layer F.Cu) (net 9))
 (segment (start 153 40) (end 153 40.75) (width 0.3048) (layer F.Cu) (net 9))
 (segment (start 132.5 50.52) (end 132.5 52.5) (width 0.3048) (layer B.Cu) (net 9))
 (segment (start 132.5 52.5) (end 129 56) (width 0.3048) (layer B.Cu) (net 9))
 (segment (start 129 56) (end 129 55.2) (width 0.3048) (layer B.Cu) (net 9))
 (segment (start 112.95 48.05) (end 113 48) (width 0.3048) (layer F.Cu) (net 9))
 (segment (start 169 56) (end 172 53) (width 0.6096) (layer F.Cu) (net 7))
 (segment (start 172 51.41) (end 171.795 51.205) (width 0.6096) (layer F.Cu) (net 7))
 (segment (start 172 53) (end 172 51.41) (width 0.6096) (layer F.Cu) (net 7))
 (segment (start 169 40) (end 172 43) (width 0.6096) (layer F.Cu) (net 7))
 (segment (start 172 44.59) (end 171.795 44.795) (width 0.6096) (layer F.Cu) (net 7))
 (segment (start 172 43) (end 172 44.59) (width 0.6096) (layer F.Cu) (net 7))
 (segment (start 150 44.75) (end 148.25 44.75) (width 0.3048) (layer B.Cu) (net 7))
 (via (at 148.25 44.75) (size 0.6858) (drill 0.3302) (layers F.Cu B.Cu) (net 7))
 (segment (start 147.25 44.75) (end 148.25 44.75) (width 0.3048) (layer B.Cu) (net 7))
 (segment (start 147.25 44.75) (end 145 42.5) (width 0.3048) (layer B.Cu) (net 7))
 (segment (start 171.795 48) (end 171.795 44.795) (width 0.6096) (layer F.Cu) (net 7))
 (segment (start 171.75 44.75) (end 150 44.75) (width 0.6096) (layer B.Cu) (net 7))
 (via (at 171.75 44.75) (size 0.6858) (drill 0.3302) (layers F.Cu B.Cu) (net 7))
 (segment (start 171.795 44.795) (end 171.75 44.75) (width 0.6096) (layer F.Cu) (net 7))
 (via (at 150 44.75) (size 0.6858) (drill 0.3302) (layers F.Cu B.Cu) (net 7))
 (segment (start 150.205 44.955) (end 150.205 48) (width 0.6096) (layer F.Cu) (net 7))
 (segment (start 150 44.75) (end 150.205 44.955) (width 0.6096) (layer F.Cu) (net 7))
 (segment (start 171.795 48) (end 171.795 51.205) (width 0.6096) (layer F.Cu) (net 7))
 (segment (start 150.205 50.955) (end 150.205 48) (width 0.6096) (layer F.Cu) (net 7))
 (segment (start 150.25 51) (end 150.205 50.955) (width 0.6096) (layer F.Cu) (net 7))
 (via (at 150.25 51) (size 0.6858) (drill 0.3302) (layers F.Cu B.Cu) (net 7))
 (segment (start 171.5 51) (end 150.25 51) (width 0.6096) (layer B.Cu) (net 7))
 (segment (start 171.75 51.25) (end 171.5 51) (width 0.6096) (layer B.Cu) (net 7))
 (via (at 171.75 51.25) (size 0.6858) (drill 0.3302) (layers F.Cu B.Cu) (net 7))
 (segment (start 171.795 51.205) (end 171.75 51.25) (width 0.6096) (layer F.Cu) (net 7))
 (segment (start 145 40) (end 145 42.5) (width 0.3048) (layer B.Cu) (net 7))
 (segment (start 140.12 42.9) (end 142.1 42.9) (width 0.3048) (layer B.Cu) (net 7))
 (segment (start 142.1 42.9) (end 145 40) (width 0.3048) (layer B.Cu) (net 7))
 (segment (start 140.25 40.75) (end 140.25 42.77) (width 0.3048) (layer F.Cu) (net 7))
 (segment (start 140.25 42.77) (end 140.12 42.9) (width 0.3048) (layer F.Cu) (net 7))
 (segment (start 115.215076 42.315076) (end 116.3 43.4) (width 0.3048) (layer F.Cu) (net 2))
 (segment (start 114.9 52.3) (end 113.05 52.3) (width 0.3048) (layer F.Cu) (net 2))
 (segment (start 116.7 50.5) (end 114.9 52.3) (width 0.3048) (layer F.Cu) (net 2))
 (via (at 116.7 50.5) (size 0.6858) (drill 0.3302) (layers F.Cu B.Cu) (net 2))
 (segment (start 116.7 43.8) (end 116.7 50.5) (width 0.3048) (layer B.Cu) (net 2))
 (segment (start 116.3 43.4) (end 116.7 43.8) (width 0.3048) (layer B.Cu) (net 2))
 (via (at 116.3 43.4) (size 0.6858) (drill 0.3302) (layers F.Cu B.Cu) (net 2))
 (segment (start 115.215076 42.115076) (end 115.215076 42.315076) (width 0.3048) (layer F.Cu) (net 2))
 (segment (start 129 48) (end 132.48 48) (width 0.3048) (layer F.Cu) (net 8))
 (segment (start 132.48 48) (end 132.5 47.98) (width 0.3048) (layer F.Cu) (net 8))
 (segment (start 116.275736 41.054416) (end 116.275736 39.774264) (width 0.3048) (layer F.Cu) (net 1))
 (segment (start 116.275736 39.774264) (end 116.5 39.55) (width 0.3048) (layer F.Cu) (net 1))
 (segment (start 116.275736 39.674264) (end 116.5 39.45) (width 0.3048) (layer F.Cu) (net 1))
 (segment (start 116.781802 39.731802) (end 116.5 39.45) (width 0.3048) (layer F.Cu) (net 1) (status 30))
 (segment (start 114.154416 43.175736) (end 112.974264 43.175736) (width 0.3048) (layer F.Cu) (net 3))
 (segment (start 112.974264 43.175736) (end 112.55 43.6) (width 0.3048) (layer F.Cu) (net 3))
 (segment (start 112.8 43.5) (end 112.45 43.5) (width 0.3048) (layer F.Cu) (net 3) (status 30))
 (segment (start 118.114214 45.014214) (end 118.114214 45.114214) (width 0.3048) (layer F.Cu) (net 5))
 (segment (start 118.114214 45.114214) (end 121 48) (width 0.3048) (layer F.Cu) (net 5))
 (segment (start 145 48) (end 145 47) (width 0.3048) (layer B.Cu) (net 5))
 (segment (start 145 47) (end 142.25 44.25) (width 0.3048) (layer B.Cu) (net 5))
 (segment (start 124.25 44) (end 121 47.25) (width 0.3048) (layer B.Cu) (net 5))
 (via (at 124.25 44) (size 0.6858) (drill 0.3302) (layers F.Cu B.Cu) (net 5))
 (segment (start 125.75 44) (end 124.25 44) (width 0.3048) (layer F.Cu) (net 5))
 (via (at 125.75 44) (size 0.6858) (drill 0.3302) (layers F.Cu B.Cu) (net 5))
 (segment (start 126.75 44) (end 125.75 44) (width 0.3048) (layer B.Cu) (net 5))
 (segment (start 127 44.25) (end 126.75 44) (width 0.3048) (layer B.Cu) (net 5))
 (segment (start 142.25 44.25) (end 127 44.25) (width 0.3048) (layer B.Cu) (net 5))
 (segment (start 121 47.25) (end 121 48) (width 0.3048) (layer B.Cu) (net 5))
 (segment (start 140.12 47.98) (end 144.98 47.98) (width 0.3048) (layer B.Cu) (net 5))
 (segment (start 144.98 47.98) (end 145 48) (width 0.3048) (layer B.Cu) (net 5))
 (segment (start 144.98 47.98) (end 145 48) (width 0.3048) (layer F.Cu) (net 5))
 (segment (start 145 48) (end 145 47.4) (width 0.3048) (layer B.Cu) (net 5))
 (segment (start 121 46.1) (end 121 48) (width 0.3048) (layer B.Cu) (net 5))
 (segment (start 119.174874 43.953553) (end 119.174874 41.825126) (width 0.3048) (layer F.Cu) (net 6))
 (segment (start 119.174874 41.825126) (end 121 40) (width 0.3048) (layer F.Cu) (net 6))
 (segment (start 129 40) (end 129 40.75) (width 0.3048) (layer B.Cu) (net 6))
 (segment (start 129 40.75) (end 126.75 43) (width 0.3048) (layer B.Cu) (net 6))
 (segment (start 124.25 43) (end 121.25 40) (width 0.3048) (layer B.Cu) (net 6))
 (via (at 124.25 43) (size 0.6858) (drill 0.3302) (layers F.Cu B.Cu) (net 6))
 (segment (start 125.75 43) (end 124.25 43) (width 0.3048) (layer F.Cu) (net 6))
 (via (at 125.75 43) (size 0.6858) (drill 0.3302) (layers F.Cu B.Cu) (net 6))
 (segment (start 126.75 43) (end 125.75 43) (width 0.3048) (layer B.Cu) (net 6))
 (segment (start 121.25 40) (end 121 40) (width 0.3048) (layer B.Cu) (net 6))
 (segment (start 140.12 50.52) (end 139.08 50.52) (width 0.3048) (layer F.Cu) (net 6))
 (segment (start 132.5 40) (end 129 40) (width 0.3048) (layer F.Cu) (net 6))
 (segment (start 133.9 41.4) (end 132.5 40) (width 0.3048) (layer F.Cu) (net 6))
 (segment (start 133.9 49.6) (end 133.9 41.4) (width 0.3048) (layer F.Cu) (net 6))
 (segment (start 135.5 51.2) (end 133.9 49.6) (width 0.3048) (layer F.Cu) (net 6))
 (segment (start 138.4 51.2) (end 135.5 51.2) (width 0.3048) (layer F.Cu) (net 6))
 (segment (start 139.08 50.52) (end 138.4 51.2) (width 0.3048) (layer F.Cu) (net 6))
 (segment (start 118.873833 42.126167) (end 121 40) (width 0.3048) (layer F.Cu) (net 6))
 (segment (start 121 56) (end 120 56) (width 0.3048) (layer F.Cu) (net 4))
 (segment (start 120 56) (end 117.4 53.4) (width 0.3048) (layer F.Cu) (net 4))
 (segment (start 117.4 53.4) (end 117.4 46.421321) (width 0.3048) (layer F.Cu) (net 4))
 (segment (start 117.4 46.421321) (end 117.053553 46.074874) (width 0.3048) (layer F.Cu) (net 4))
 (segment (start 140.725 52.025) (end 126.775 52.025) (width 0.3048) (layer F.Cu) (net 4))
 (segment (start 123.25 51.25) (end 121 53.5) (width 0.3048) (layer F.Cu) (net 4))
 (segment (start 124 51.25) (end 123.25 51.25) (width 0.3048) (layer F.Cu) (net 4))
 (segment (start 124.25 51) (end 124 51.25) (width 0.3048) (layer F.Cu) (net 4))
 (via (at 124.25 51) (size 0.6858) (drill 0.3302) (layers F.Cu B.Cu) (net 4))
 (segment (start 125.75 51) (end 124.25 51) (width 0.3048) (layer B.Cu) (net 4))
 (via (at 125.75 51) (size 0.6858) (drill 0.3302) (layers F.Cu B.Cu) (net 4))
 (segment (start 126.775 52.025) (end 125.75 51) (width 0.3048) (layer F.Cu) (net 4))
 (segment (start 121 53.5) (end 121 56) (width 0.3048) (layer F.Cu) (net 4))
 (segment (start 145 56) (end 144.9 56) (width 0.3048) (layer F.Cu) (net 4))
 (segment (start 144.9 56) (end 141.4 52.5) (width 0.3048) (layer F.Cu) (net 4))
 (segment (start 141.4 46.72) (end 140.12 45.44) (width 0.3048) (layer F.Cu) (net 4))
 (segment (start 141.4 52.5) (end 141.4 46.72) (width 0.3048) (layer F.Cu) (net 4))
 (segment (start 145 56) (end 144.7 56) (width 0.3048) (layer F.Cu) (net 4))
 (segment (start 144.7 56) (end 140.725 52.025) (width 0.3048) (layer F.Cu) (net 4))
 (segment (start 140.725 52.025) (end 140.7 52) (width 0.3048) (layer F.Cu) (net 4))
 (segment (start 140.12 45.44) (end 139.84 45.44) (width 0.3048) (layer F.Cu) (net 4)))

